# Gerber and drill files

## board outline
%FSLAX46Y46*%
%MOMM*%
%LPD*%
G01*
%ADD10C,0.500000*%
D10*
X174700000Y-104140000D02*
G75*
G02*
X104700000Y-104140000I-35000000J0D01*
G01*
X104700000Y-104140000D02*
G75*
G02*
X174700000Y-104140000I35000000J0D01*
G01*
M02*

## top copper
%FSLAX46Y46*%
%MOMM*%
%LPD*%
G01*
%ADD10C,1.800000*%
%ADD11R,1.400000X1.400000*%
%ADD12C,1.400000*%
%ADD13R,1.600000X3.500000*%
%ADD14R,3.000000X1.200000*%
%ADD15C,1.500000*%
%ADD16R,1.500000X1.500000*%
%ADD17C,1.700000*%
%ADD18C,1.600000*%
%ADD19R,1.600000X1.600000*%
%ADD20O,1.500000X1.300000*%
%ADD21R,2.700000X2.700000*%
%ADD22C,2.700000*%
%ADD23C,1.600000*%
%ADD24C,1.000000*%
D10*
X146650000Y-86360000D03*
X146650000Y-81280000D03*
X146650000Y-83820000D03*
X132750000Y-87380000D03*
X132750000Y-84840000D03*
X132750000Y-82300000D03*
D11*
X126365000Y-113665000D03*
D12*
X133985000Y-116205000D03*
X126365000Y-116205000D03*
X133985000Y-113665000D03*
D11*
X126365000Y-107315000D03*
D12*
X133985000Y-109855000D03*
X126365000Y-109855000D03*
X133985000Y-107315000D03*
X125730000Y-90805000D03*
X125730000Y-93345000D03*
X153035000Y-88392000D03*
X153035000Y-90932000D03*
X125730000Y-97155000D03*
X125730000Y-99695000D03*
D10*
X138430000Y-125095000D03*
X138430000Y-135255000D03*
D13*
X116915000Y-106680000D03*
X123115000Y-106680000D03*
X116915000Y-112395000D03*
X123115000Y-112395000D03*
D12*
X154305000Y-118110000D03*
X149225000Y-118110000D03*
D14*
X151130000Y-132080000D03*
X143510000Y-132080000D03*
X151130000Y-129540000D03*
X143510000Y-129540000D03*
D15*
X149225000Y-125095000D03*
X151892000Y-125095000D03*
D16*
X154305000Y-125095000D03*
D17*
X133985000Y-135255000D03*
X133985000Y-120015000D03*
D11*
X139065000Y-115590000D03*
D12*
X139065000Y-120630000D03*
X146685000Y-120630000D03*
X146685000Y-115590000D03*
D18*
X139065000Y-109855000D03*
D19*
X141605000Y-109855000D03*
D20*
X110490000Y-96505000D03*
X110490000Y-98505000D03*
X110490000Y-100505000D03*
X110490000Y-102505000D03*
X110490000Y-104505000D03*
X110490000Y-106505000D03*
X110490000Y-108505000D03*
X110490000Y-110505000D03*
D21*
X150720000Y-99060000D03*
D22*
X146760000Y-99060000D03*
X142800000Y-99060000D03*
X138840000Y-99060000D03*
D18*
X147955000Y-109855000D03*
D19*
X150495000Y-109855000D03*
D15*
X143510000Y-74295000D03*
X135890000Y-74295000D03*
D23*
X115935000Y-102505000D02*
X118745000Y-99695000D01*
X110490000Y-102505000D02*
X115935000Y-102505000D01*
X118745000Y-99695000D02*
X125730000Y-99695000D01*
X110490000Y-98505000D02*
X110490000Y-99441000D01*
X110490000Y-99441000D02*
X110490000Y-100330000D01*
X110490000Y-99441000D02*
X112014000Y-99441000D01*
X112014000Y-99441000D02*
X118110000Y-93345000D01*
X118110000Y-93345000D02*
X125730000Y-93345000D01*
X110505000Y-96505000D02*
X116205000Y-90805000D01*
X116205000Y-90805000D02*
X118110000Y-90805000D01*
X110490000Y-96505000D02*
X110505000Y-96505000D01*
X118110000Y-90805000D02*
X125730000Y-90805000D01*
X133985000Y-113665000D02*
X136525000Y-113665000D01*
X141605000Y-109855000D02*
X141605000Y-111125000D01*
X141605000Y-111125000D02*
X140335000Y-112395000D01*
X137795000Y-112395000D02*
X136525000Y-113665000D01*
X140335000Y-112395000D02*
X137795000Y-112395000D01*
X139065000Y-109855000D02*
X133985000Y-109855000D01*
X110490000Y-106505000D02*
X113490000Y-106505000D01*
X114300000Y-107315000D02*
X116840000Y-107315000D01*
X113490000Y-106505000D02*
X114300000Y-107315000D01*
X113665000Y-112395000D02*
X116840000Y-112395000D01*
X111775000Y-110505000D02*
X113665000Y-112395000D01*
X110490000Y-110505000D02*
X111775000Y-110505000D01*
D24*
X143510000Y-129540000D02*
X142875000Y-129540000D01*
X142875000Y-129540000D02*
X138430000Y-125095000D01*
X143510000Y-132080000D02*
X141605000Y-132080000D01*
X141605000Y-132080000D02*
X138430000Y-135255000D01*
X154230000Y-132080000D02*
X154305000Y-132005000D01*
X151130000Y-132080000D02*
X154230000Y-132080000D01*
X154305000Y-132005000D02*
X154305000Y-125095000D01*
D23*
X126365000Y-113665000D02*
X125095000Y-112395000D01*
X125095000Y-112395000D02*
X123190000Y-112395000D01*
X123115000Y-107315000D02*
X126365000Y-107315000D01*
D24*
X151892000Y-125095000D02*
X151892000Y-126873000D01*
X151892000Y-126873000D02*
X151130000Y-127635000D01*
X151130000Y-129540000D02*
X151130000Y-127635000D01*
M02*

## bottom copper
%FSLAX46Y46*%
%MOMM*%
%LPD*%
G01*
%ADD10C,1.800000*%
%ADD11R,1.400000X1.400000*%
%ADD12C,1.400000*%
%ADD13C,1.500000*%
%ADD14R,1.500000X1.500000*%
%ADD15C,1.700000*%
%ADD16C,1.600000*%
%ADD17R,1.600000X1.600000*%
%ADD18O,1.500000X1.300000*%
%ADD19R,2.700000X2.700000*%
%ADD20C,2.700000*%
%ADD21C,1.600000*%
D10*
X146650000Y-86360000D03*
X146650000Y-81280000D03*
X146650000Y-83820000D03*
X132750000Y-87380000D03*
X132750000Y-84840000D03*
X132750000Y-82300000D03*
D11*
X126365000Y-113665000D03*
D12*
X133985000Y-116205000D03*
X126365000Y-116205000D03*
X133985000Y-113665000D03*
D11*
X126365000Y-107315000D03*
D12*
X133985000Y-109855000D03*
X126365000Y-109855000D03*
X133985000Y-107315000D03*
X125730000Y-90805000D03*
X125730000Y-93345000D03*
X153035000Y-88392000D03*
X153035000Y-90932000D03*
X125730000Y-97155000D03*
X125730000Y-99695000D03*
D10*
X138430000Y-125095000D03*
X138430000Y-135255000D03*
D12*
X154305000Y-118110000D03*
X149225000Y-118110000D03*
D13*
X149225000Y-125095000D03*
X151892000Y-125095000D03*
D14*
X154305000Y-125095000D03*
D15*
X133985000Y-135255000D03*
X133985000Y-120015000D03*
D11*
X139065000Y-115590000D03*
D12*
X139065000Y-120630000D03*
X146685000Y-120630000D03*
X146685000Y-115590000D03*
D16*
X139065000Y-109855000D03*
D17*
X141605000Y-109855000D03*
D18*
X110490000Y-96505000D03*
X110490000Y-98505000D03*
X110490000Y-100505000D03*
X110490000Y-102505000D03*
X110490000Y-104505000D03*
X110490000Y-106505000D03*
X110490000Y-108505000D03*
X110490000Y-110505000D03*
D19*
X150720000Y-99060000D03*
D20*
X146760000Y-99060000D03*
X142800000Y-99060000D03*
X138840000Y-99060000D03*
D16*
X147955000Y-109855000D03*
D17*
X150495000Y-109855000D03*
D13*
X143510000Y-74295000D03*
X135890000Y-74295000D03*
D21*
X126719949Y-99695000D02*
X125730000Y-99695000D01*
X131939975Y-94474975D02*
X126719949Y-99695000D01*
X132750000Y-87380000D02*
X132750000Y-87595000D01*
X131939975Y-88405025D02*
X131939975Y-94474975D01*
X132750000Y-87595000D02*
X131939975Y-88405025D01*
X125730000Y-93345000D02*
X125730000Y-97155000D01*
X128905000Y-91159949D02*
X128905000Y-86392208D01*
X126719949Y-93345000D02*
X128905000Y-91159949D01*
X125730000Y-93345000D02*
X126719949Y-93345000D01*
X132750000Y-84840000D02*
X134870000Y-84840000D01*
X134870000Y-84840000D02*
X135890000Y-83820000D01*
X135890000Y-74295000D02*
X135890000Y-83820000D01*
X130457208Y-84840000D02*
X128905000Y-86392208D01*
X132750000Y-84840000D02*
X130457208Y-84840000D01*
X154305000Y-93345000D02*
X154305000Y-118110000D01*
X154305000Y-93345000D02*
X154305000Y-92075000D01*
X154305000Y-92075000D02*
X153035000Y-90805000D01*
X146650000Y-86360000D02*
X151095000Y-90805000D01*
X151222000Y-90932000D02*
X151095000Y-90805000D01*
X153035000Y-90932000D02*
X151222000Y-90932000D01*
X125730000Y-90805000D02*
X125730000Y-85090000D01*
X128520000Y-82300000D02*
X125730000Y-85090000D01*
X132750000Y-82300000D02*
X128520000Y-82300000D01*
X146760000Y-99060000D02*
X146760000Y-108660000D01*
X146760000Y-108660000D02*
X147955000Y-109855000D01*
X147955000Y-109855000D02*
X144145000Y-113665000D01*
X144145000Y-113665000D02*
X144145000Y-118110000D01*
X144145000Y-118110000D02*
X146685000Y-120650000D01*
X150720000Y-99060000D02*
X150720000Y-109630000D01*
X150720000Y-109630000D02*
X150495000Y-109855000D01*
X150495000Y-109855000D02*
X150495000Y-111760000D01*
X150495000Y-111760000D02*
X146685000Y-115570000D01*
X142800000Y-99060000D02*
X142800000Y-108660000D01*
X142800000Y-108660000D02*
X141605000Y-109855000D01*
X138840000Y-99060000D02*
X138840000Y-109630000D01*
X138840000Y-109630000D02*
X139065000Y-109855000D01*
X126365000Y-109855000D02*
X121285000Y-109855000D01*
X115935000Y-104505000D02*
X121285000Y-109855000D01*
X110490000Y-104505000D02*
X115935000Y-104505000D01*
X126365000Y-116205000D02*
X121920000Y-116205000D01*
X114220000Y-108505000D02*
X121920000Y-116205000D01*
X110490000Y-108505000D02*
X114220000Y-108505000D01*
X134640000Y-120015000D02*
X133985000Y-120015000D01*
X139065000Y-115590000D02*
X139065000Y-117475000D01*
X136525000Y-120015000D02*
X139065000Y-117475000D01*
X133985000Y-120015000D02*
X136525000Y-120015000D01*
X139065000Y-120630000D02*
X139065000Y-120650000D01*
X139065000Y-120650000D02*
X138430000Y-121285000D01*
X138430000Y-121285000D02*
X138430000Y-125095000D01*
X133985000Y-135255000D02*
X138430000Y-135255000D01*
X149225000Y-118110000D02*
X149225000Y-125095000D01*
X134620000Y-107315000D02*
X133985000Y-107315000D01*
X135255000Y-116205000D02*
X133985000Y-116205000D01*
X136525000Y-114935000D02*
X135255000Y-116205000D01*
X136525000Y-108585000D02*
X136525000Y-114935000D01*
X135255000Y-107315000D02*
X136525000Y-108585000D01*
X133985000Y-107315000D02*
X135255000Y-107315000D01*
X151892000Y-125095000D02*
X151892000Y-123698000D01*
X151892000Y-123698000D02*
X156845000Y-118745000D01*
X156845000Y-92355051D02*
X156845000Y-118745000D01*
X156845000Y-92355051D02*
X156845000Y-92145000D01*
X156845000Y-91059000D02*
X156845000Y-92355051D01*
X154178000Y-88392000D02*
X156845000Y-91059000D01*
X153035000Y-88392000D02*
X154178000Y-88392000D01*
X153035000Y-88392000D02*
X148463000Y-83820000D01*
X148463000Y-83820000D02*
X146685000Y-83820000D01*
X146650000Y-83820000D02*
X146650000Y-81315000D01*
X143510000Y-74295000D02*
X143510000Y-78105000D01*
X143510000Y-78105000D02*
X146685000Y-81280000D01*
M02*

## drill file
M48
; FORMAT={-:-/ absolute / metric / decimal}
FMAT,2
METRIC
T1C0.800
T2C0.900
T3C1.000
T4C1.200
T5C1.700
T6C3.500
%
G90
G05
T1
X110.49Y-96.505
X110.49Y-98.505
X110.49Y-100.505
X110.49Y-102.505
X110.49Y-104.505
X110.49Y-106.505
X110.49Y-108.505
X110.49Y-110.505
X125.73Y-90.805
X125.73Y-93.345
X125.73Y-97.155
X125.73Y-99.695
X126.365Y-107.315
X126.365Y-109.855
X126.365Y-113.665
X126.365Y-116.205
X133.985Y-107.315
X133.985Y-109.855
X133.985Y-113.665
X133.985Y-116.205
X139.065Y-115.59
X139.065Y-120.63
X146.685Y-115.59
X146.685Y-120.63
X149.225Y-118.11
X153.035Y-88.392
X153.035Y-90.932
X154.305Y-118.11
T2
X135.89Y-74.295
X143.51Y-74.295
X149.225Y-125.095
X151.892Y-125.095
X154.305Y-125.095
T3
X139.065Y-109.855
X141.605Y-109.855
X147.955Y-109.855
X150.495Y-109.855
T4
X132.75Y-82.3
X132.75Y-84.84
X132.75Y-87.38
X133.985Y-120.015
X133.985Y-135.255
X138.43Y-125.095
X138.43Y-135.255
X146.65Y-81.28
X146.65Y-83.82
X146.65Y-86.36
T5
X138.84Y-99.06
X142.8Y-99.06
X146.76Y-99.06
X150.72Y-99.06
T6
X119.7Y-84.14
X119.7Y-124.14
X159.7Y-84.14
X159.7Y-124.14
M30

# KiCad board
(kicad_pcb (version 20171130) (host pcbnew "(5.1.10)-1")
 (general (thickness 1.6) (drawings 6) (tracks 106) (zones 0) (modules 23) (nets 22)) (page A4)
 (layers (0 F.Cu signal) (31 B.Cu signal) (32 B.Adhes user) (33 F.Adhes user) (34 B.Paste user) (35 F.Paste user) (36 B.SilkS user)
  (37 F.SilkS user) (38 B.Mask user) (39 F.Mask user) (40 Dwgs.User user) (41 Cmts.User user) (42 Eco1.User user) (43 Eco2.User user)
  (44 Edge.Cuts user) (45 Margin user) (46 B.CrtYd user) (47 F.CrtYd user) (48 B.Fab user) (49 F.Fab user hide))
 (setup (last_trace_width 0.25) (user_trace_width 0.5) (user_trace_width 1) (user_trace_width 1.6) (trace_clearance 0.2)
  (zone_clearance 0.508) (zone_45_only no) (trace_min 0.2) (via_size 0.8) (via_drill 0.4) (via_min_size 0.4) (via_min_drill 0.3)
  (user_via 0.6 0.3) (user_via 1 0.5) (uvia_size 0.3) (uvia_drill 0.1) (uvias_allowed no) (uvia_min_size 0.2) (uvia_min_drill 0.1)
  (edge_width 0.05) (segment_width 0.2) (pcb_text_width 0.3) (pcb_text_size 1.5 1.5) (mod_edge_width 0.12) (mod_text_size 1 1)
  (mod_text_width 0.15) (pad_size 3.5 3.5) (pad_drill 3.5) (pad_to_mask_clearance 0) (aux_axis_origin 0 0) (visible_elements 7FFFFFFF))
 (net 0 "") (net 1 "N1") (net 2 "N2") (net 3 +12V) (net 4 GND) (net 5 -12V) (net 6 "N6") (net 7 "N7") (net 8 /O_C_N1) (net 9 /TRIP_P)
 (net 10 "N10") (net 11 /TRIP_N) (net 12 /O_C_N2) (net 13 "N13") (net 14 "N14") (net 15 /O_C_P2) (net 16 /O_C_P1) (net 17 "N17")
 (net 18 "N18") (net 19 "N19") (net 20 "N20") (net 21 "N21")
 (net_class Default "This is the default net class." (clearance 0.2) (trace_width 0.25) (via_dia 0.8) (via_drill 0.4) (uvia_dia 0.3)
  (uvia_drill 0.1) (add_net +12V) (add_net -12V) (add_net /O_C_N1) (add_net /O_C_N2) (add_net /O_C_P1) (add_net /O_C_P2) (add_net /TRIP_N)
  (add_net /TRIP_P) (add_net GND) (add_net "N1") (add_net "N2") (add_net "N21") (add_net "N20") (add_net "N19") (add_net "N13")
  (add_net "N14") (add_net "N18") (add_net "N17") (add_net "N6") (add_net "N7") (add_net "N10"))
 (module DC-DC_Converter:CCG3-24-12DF (layer F.Cu) (at 139.7 83.82)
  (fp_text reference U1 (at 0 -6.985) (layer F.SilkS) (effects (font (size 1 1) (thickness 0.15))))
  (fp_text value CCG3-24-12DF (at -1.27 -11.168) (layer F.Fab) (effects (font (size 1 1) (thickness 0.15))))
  (pad 3 thru_hole circle (at 6.95 2.54) (size 1.8 1.8) (drill 1.2) (layers *.Cu *.Mask) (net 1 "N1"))
  (pad 1 thru_hole circle (at 6.95 -2.54) (size 1.8 1.8) (drill 1.2) (layers *.Cu *.Mask) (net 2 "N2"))
  (pad 2 thru_hole circle (at 6.95 0) (size 1.8 1.8) (drill 1.2) (layers *.Cu *.Mask) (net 2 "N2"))
  (pad 6 thru_hole circle (at -6.95 3.56) (size 1.8 1.8) (drill 1.2) (layers *.Cu *.Mask) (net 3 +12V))
  (pad 5 thru_hole circle (at -6.95 1.02) (size 1.8 1.8) (drill 1.2) (layers *.Cu *.Mask) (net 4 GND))
  (pad 4 thru_hole circle (at -6.95 -1.52) (size 1.8 1.8) (drill 1.2) (layers *.Cu *.Mask) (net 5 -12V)))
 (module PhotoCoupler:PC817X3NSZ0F (layer F.Cu) (at 126.365 113.665)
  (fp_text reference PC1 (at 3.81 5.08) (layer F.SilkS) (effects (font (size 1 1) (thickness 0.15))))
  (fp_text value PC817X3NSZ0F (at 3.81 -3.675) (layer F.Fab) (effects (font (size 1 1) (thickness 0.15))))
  (pad 1 thru_hole rect (at 0 0) (size 1.4 1.4) (drill 0.8) (layers *.Cu *.Mask) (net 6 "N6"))
  (pad 3 thru_hole circle (at 7.62 2.54) (size 1.4 1.4) (drill 0.8) (layers *.Cu *.Mask) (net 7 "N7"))
  (pad 2 thru_hole circle (at 0 2.54) (size 1.4 1.4) (drill 0.8) (layers *.Cu *.Mask) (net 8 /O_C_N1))
  (pad 4 thru_hole circle (at 7.62 0) (size 1.4 1.4) (drill 0.8) (layers *.Cu *.Mask) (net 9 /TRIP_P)))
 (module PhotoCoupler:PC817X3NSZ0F (layer F.Cu) (at 126.365 107.315)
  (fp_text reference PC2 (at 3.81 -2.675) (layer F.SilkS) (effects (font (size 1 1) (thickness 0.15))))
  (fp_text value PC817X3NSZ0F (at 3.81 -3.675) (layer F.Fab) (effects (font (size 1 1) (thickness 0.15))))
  (pad 1 thru_hole rect (at 0 0) (size 1.4 1.4) (drill 0.8) (layers *.Cu *.Mask) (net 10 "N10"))
  (pad 3 thru_hole circle (at 7.62 2.54) (size 1.4 1.4) (drill 0.8) (layers *.Cu *.Mask) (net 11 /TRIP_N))
  (pad 2 thru_hole circle (at 0 2.54) (size 1.4 1.4) (drill 0.8) (layers *.Cu *.Mask) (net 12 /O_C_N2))
  (pad 4 thru_hole circle (at 7.62 0) (size 1.4 1.4) (drill 0.8) (layers *.Cu *.Mask) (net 7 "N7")))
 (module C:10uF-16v (layer F.Cu) (at 125.73 92.075 90)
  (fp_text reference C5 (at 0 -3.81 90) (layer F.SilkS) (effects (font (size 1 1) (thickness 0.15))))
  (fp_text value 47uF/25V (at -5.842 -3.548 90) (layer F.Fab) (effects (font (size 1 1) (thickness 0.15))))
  (pad 2 thru_hole circle (at 1.27 0 90) (size 1.4 1.4) (drill 0.8) (layers *.Cu *.Mask) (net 5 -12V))
  (pad 1 thru_hole circle (at -1.27 0 90) (size 1.4 1.4) (drill 0.8) (layers *.Cu *.Mask) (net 4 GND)))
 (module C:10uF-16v (layer F.Cu) (at 153.035 89.662 90)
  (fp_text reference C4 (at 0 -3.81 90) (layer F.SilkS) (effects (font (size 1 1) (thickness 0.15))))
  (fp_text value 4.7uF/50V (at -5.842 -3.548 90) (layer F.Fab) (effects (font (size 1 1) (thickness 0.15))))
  (pad 2 thru_hole circle (at 1.27 0 90) (size 1.4 1.4) (drill 0.8) (layers *.Cu *.Mask) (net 2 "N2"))
  (pad 1 thru_hole circle (at -1.27 0 90) (size 1.4 1.4) (drill 0.8) (layers *.Cu *.Mask) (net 1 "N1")))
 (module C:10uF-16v (layer F.Cu) (at 125.73 98.425 90)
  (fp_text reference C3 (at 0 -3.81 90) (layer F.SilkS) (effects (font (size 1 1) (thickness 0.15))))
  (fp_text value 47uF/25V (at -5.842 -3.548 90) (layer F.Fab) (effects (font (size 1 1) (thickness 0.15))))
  (pad 2 thru_hole circle (at 1.27 0 90) (size 1.4 1.4) (drill 0.8) (layers *.Cu *.Mask) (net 4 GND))
  (pad 1 thru_hole circle (at -1.27 0 90) (size 1.4 1.4) (drill 0.8) (layers *.Cu *.Mask) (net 3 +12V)))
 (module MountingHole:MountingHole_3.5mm (layer F.Cu) (at 119.7 84.14)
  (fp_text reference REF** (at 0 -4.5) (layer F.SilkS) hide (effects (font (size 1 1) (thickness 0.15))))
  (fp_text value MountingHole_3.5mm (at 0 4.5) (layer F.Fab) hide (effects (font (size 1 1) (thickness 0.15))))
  (pad 1 np_thru_hole circle (at 0 0) (size 3.5 3.5) (drill 3.5) (layers *.Cu *.Mask)))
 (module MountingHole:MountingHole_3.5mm (layer F.Cu) (at 119.7 124.14)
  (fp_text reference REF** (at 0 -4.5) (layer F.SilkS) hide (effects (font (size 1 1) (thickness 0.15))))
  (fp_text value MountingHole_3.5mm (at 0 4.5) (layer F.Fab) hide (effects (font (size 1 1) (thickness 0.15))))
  (pad 1 np_thru_hole circle (at 0 0) (size 3.5 3.5) (drill 3.5) (layers *.Cu *.Mask)))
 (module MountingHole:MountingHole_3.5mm (layer F.Cu) (at 159.7 124.14)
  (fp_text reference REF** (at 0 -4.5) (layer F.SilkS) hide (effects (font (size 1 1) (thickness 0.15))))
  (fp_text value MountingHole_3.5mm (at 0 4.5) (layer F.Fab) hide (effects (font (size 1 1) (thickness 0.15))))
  (pad 1 np_thru_hole circle (at 0 0) (size 3.5 3.5) (drill 3.5) (layers *.Cu *.Mask)))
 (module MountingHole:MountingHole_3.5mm (layer F.Cu) (at 159.7 84.14)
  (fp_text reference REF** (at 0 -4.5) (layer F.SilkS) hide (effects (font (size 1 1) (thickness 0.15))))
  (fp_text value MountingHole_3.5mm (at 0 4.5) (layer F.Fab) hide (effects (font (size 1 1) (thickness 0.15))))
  (pad 1 np_thru_hole circle (at 0 0) (size 3.5 3.5) (drill 3.5) (layers *.Cu *.Mask)))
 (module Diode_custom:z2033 (layer F.Cu) (at 138.43 130.175 90)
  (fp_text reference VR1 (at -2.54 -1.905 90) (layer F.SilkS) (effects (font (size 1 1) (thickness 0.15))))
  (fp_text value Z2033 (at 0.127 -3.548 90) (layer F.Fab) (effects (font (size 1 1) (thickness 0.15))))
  (pad 2 thru_hole circle (at 5.08 0 90) (size 1.8 1.8) (drill 1.2) (layers *.Cu *.Mask) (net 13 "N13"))
  (pad 1 thru_hole circle (at -5.08 0 90) (size 1.8 1.8) (drill 1.2) (layers *.Cu *.Mask) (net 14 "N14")))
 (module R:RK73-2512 (layer F.Cu) (at 120.015 106.68)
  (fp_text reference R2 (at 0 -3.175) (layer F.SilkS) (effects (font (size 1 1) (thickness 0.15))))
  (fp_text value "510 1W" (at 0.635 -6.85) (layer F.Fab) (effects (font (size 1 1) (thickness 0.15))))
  (pad 1 smd rect (at -3.1 0) (size 1.6 3.5) (layers F.Cu F.Paste F.Mask) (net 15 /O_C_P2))
  (pad 2 smd rect (at 3.1 0) (size 1.6 3.5) (layers F.Cu F.Paste F.Mask) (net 10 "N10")))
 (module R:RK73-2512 (layer F.Cu) (at 120.015 112.395)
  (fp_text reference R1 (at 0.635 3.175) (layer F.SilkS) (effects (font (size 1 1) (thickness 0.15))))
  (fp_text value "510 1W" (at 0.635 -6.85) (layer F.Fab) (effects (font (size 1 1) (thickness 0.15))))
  (pad 1 smd rect (at -3.1 0) (size 1.6 3.5) (layers F.Cu F.Paste F.Mask) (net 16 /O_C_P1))
  (pad 2 smd rect (at 3.1 0) (size 1.6 3.5) (layers F.Cu F.Paste F.Mask) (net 6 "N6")))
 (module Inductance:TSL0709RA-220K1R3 (layer F.Cu) (at 151.765 118.11)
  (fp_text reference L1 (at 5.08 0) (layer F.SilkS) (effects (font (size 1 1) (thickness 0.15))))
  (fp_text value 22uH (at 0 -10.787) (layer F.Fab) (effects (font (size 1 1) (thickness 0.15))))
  (pad 2 thru_hole circle (at 2.54 0) (size 1.4 1.4) (drill 0.8) (layers *.Cu *.Mask) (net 1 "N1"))
  (pad 1 thru_hole circle (at -2.54 0) (size 1.4 1.4) (drill 0.8) (layers *.Cu *.Mask) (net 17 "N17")))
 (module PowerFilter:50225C (layer F.Cu) (at 147.32 130.81)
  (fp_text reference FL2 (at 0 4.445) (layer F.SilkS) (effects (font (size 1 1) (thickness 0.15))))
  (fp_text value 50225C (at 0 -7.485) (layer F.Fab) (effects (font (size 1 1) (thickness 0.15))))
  (pad 3 smd rect (at 3.81 1.27) (size 3 1.2) (layers F.Cu F.Paste F.Mask) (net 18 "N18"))
  (pad 2 smd rect (at -3.81 1.27) (size 3 1.2) (layers F.Cu F.Paste F.Mask) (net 14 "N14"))
  (pad 4 smd rect (at 3.81 -1.27) (size 3 1.2) (layers F.Cu F.Paste F.Mask) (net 2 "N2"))
  (pad 1 smd rect (at -3.81 -1.27) (size 3 1.2) (layers F.Cu F.Paste F.Mask) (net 13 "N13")))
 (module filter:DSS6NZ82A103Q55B (layer F.Cu) (at 151.765 125.095 180)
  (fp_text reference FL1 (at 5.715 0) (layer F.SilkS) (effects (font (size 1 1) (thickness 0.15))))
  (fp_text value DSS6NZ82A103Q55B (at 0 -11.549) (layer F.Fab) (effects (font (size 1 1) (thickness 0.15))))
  (pad 3 thru_hole circle (at 2.54 0 180) (size 1.5 1.5) (drill 0.9) (layers *.Cu *.Mask) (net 17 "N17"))
  (pad 2 thru_hole circle (at -0.127 0 180) (size 1.5 1.5) (drill 0.9) (layers *.Cu *.Mask) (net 2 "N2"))
  (pad 1 thru_hole rect (at -2.54 0 180) (size 1.5 1.5) (drill 0.9) (layers *.Cu *.Mask) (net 18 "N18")))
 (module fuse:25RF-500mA (layer F.Cu) (at 133.985 127.635 270)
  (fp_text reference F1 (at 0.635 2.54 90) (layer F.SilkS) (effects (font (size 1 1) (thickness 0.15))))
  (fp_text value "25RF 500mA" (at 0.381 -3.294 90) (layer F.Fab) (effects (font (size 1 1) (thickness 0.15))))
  (pad 2 thru_hole circle (at 7.62 0 270) (size 1.7 1.7) (drill 1.2) (layers *.Cu *.Mask) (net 14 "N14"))
  (pad 1 thru_hole circle (at -7.62 0 270) (size 1.7 1.7) (drill 1.2) (layers *.Cu *.Mask) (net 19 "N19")))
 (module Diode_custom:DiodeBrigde (layer F.Cu) (at 142.875 118.11)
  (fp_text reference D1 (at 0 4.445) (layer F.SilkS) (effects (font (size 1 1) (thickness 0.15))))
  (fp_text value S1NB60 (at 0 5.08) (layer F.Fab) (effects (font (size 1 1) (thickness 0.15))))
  (pad 1 thru_hole rect (at -3.81 -2.52) (size 1.4 1.4) (drill 0.8) (layers *.Cu *.Mask) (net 19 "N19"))
  (pad 4 thru_hole circle (at -3.81 2.52) (size 1.4 1.4) (drill 0.8) (layers *.Cu *.Mask) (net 13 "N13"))
  (pad 3 thru_hole circle (at 3.81 2.52) (size 1.4 1.4) (drill 0.8) (layers *.Cu *.Mask) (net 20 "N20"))
  (pad 2 thru_hole circle (at 3.81 -2.52) (size 1.4 1.4) (drill 0.8) (layers *.Cu *.Mask) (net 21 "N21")))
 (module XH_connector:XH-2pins (layer F.Cu) (at 140.208 109.855 270)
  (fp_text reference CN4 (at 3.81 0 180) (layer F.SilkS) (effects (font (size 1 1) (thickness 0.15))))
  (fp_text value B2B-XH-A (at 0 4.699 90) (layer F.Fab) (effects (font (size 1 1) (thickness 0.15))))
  (pad 2 thru_hole circle (at 0 1.143 270) (size 1.6 1.6) (drill 1) (layers *.Cu *.Mask) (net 11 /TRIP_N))
  (pad 1 thru_hole rect (at 0 -1.397 270) (size 1.6 1.6) (drill 1) (layers *.Cu *.Mask) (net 9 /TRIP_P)))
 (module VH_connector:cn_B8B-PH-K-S (layer F.Cu) (at 110.49 103.505 90)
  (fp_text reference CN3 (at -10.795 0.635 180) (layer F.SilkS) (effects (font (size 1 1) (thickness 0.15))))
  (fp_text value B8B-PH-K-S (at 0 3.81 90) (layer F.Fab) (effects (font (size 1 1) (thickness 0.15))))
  (pad 8 thru_hole oval (at 7 0 90) (size 1.3 1.5) (drill 0.8) (layers *.Cu *.Mask) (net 5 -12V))
  (pad 7 thru_hole oval (at 5 0 90) (size 1.3 1.5) (drill 0.8) (layers *.Cu *.Mask) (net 4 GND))
  (pad 6 thru_hole oval (at 3 0 90) (size 1.3 1.5) (drill 0.8) (layers *.Cu *.Mask) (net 4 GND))
  (pad 5 thru_hole oval (at 1 0 90) (size 1.3 1.5) (drill 0.8) (layers *.Cu *.Mask) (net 3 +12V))
  (pad 4 thru_hole oval (at -1 0 90) (size 1.3 1.5) (drill 0.8) (layers *.Cu *.Mask) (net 12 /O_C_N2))
  (pad 3 thru_hole oval (at -3 0 90) (size 1.3 1.5) (drill 0.8) (layers *.Cu *.Mask) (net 15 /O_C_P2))
  (pad 2 thru_hole oval (at -5 0 90) (size 1.3 1.5) (drill 0.8) (layers *.Cu *.Mask) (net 8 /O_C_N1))
  (pad 1 thru_hole oval (at -7 0 90) (size 1.3 1.5) (drill 0.8) (layers *.Cu *.Mask) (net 16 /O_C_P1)))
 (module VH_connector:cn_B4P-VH (layer F.Cu) (at 144.78 99.06 180)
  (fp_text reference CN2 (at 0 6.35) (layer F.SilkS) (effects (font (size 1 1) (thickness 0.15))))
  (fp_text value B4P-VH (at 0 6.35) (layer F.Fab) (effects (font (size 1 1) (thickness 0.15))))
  (pad 1 thru_hole rect (at -5.94 0 180) (size 2.7 2.7) (drill 1.7) (layers *.Cu *.Mask) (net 21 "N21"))
  (pad 2 thru_hole circle (at -1.98 0 180) (size 2.7 2.7) (drill 1.7) (layers *.Cu *.Mask) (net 20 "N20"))
  (pad 3 thru_hole circle (at 1.98 0 180) (size 2.7 2.7) (drill 1.7) (layers *.Cu *.Mask) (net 9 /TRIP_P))
  (pad 4 thru_hole circle (at 5.94 0 180) (size 2.7 2.7) (drill 1.7) (layers *.Cu *.Mask) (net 11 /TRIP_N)))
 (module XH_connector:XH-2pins (layer F.Cu) (at 149.098 109.855 270)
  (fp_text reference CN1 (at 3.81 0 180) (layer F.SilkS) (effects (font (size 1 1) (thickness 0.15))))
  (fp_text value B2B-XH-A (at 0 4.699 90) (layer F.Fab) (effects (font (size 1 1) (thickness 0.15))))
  (pad 2 thru_hole circle (at 0 1.143 270) (size 1.6 1.6) (drill 1) (layers *.Cu *.Mask) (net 20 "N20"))
  (pad 1 thru_hole rect (at 0 -1.397 270) (size 1.6 1.6) (drill 1) (layers *.Cu *.Mask) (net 21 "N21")))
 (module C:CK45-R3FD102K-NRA (layer F.Cu) (at 139.7 74.295)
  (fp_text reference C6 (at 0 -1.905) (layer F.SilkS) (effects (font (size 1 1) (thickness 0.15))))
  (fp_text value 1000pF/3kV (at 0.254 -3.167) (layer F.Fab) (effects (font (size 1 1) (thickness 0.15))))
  (pad 2 thru_hole circle (at 3.81 0) (size 1.5 1.5) (drill 0.9) (layers *.Cu *.Mask) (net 2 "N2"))
  (pad 1 thru_hole circle (at -3.81 0) (size 1.5 1.5) (drill 0.9) (layers *.Cu *.Mask) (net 4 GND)))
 (gr_circle (center 139.7 104.14) (end 174.7 104.14) (layer Edge.Cuts) (width 0.5))
 (segment (start 115.935 102.505) (end 118.745 99.695) (width 1.6) (layer F.Cu) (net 3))
 (segment (start 110.49 102.505) (end 115.935 102.505) (width 1.6) (layer F.Cu) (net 3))
 (segment (start 126.719949 99.695) (end 125.73 99.695) (width 1.6) (layer B.Cu) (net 3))
 (segment (start 118.745 99.695) (end 125.73 99.695) (width 1.6) (layer F.Cu) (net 3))
 (segment (start 131.939975 94.474975) (end 126.719949 99.695) (width 1.6) (layer B.Cu) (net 3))
 (segment (start 132.75 87.38) (end 132.75 87.595) (width 1.6) (layer B.Cu) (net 3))
 (segment (start 131.939975 88.405025) (end 131.939975 94.474975) (width 1.6) (layer B.Cu) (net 3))
 (segment (start 132.75 87.595) (end 131.939975 88.405025) (width 1.6) (layer B.Cu) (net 3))
 (segment (start 110.49 98.505) (end 110.49 99.441) (width 1.6) (layer F.Cu) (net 4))
 (segment (start 110.49 99.441) (end 110.49 100.33) (width 1.6) (layer F.Cu) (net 4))
 (segment (start 125.73 93.345) (end 125.73 97.155) (width 1.6) (layer B.Cu) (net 4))
 (segment (start 110.49 99.441) (end 112.014 99.441) (width 1.6) (layer F.Cu) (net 4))
 (segment (start 112.014 99.441) (end 118.11 93.345) (width 1.6) (layer F.Cu) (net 4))
 (segment (start 118.11 93.345) (end 125.73 93.345) (width 1.6) (layer F.Cu) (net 4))
 (segment (start 128.905 91.159949) (end 128.905 86.392208) (width 1.6) (layer B.Cu) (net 4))
 (segment (start 126.719949 93.345) (end 128.905 91.159949) (width 1.6) (layer B.Cu) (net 4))
 (segment (start 125.73 93.345) (end 126.719949 93.345) (width 1.6) (layer B.Cu) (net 4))
 (segment (start 132.75 84.84) (end 134.87 84.84) (width 1.6) (layer B.Cu) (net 4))
 (segment (start 134.87 84.84) (end 135.89 83.82) (width 1.6) (layer B.Cu) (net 4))
 (segment (start 135.89 74.295) (end 135.89 83.82) (width 1.6) (layer B.Cu) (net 4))
 (segment (start 130.457208 84.84) (end 128.905 86.392208) (width 1.6) (layer B.Cu) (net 4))
 (segment (start 132.75 84.84) (end 130.457208 84.84) (width 1.6) (layer B.Cu) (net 4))
 (segment (start 154.305 93.345) (end 154.305 118.11) (width 1.6) (layer B.Cu) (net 1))
 (segment (start 154.305 93.345) (end 154.305 92.075) (width 1.6) (layer B.Cu) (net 1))
 (segment (start 154.305 92.075) (end 153.035 90.805) (width 1.6) (layer B.Cu) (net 1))
 (segment (start 146.65 86.36) (end 151.095 90.805) (width 1.6) (layer B.Cu) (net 1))
 (segment (start 151.222 90.932) (end 151.095 90.805) (width 1.6) (layer B.Cu) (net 1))
 (segment (start 153.035 90.932) (end 151.222 90.932) (width 1.6) (layer B.Cu) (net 1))
 (segment (start 110.505 96.505) (end 116.205 90.805) (width 1.6) (layer F.Cu) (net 5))
 (segment (start 116.205 90.805) (end 118.11 90.805) (width 1.6) (layer F.Cu) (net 5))
 (segment (start 110.49 96.505) (end 110.505 96.505) (width 1.6) (layer F.Cu) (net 5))
 (segment (start 118.11 90.805) (end 125.73 90.805) (width 1.6) (layer F.Cu) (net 5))
 (segment (start 125.73 90.805) (end 125.73 85.09) (width 1.6) (layer B.Cu) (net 5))
 (segment (start 128.52 82.3) (end 125.73 85.09) (width 1.6) (layer B.Cu) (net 5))
 (segment (start 132.75 82.3) (end 128.52 82.3) (width 1.6) (layer B.Cu) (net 5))
 (segment (start 146.76 99.06) (end 146.76 108.66) (width 1.6) (layer B.Cu) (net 20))
 (segment (start 146.76 108.66) (end 147.955 109.855) (width 1.6) (layer B.Cu) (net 20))
 (segment (start 147.955 109.855) (end 144.145 113.665) (width 1.6) (layer B.Cu) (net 20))
 (segment (start 144.145 113.665) (end 144.145 118.11) (width 1.6) (layer B.Cu) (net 20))
 (segment (start 144.145 118.11) (end 146.685 120.65) (width 1.6) (layer B.Cu) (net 20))
 (segment (start 150.72 99.06) (end 150.72 109.63) (width 1.6) (layer B.Cu) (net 21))
 (segment (start 150.72 109.63) (end 150.495 109.855) (width 1.6) (layer B.Cu) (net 21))
 (segment (start 150.495 109.855) (end 150.495 111.76) (width 1.6) (layer B.Cu) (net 21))
 (segment (start 150.495 111.76) (end 146.685 115.57) (width 1.6) (layer B.Cu) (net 21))
 (segment (start 142.8 99.06) (end 142.8 108.66) (width 1.6) (layer B.Cu) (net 9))
 (segment (start 142.8 108.66) (end 141.605 109.855) (width 1.6) (layer B.Cu) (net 9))
 (segment (start 133.985 113.665) (end 136.525 113.665) (width 1.6) (layer F.Cu) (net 9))
 (segment (start 141.605 109.855) (end 141.605 111.125) (width 1.6) (layer F.Cu) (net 9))
 (segment (start 141.605 111.125) (end 140.335 112.395) (width 1.6) (layer F.Cu) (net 9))
 (segment (start 137.795 112.395) (end 136.525 113.665) (width 1.6) (layer F.Cu) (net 9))
 (segment (start 140.335 112.395) (end 137.795 112.395) (width 1.6) (layer F.Cu) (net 9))
 (segment (start 138.84 99.06) (end 138.84 109.63) (width 1.6) (layer B.Cu) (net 11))
 (segment (start 138.84 109.63) (end 139.065 109.855) (width 1.6) (layer B.Cu) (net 11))
 (segment (start 139.065 109.855) (end 133.985 109.855) (width 1.6) (layer F.Cu) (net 11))
 (segment (start 126.365 109.855) (end 121.285 109.855) (width 1.6) (layer B.Cu) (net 12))
 (segment (start 115.935 104.505) (end 121.285 109.855) (width 1.6) (layer B.Cu) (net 12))
 (segment (start 110.49 104.505) (end 115.935 104.505) (width 1.6) (layer B.Cu) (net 12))
 (segment (start 110.49 106.505) (end 113.49 106.505) (width 1.6) (layer F.Cu) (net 15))
 (segment (start 114.3 107.315) (end 116.84 107.315) (width 1.6) (layer F.Cu) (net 15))
 (segment (start 113.49 106.505) (end 114.3 107.315) (width 1.6) (layer F.Cu) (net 15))
 (segment (start 126.365 116.205) (end 121.92 116.205) (width 1.6) (layer B.Cu) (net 8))
 (segment (start 114.22 108.505) (end 121.92 116.205) (width 1.6) (layer B.Cu) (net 8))
 (segment (start 110.49 108.505) (end 114.22 108.505) (width 1.6) (layer B.Cu) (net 8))
 (segment (start 113.665 112.395) (end 116.84 112.395) (width 1.6) (layer F.Cu) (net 16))
 (segment (start 111.775 110.505) (end 113.665 112.395) (width 1.6) (layer F.Cu) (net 16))
 (segment (start 110.49 110.505) (end 111.775 110.505) (width 1.6) (layer F.Cu) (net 16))
 (segment (start 134.64 120.015) (end 133.985 120.015) (width 1.6) (layer B.Cu) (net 19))
 (segment (start 139.065 115.59) (end 139.065 117.475) (width 1.6) (layer B.Cu) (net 19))
 (segment (start 136.525 120.015) (end 139.065 117.475) (width 1.6) (layer B.Cu) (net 19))
 (segment (start 133.985 120.015) (end 136.525 120.015) (width 1.6) (layer B.Cu) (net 19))
 (segment (start 143.51 129.54) (end 142.875 129.54) (width 1) (layer F.Cu) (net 13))
 (segment (start 142.875 129.54) (end 138.43 125.095) (width 1) (layer F.Cu) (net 13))
 (segment (start 139.065 120.63) (end 139.065 120.65) (width 1.6) (layer B.Cu) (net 13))
 (segment (start 139.065 120.65) (end 138.43 121.285) (width 1.6) (layer B.Cu) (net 13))
 (segment (start 138.43 121.285) (end 138.43 125.095) (width 1.6) (layer B.Cu) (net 13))
 (segment (start 143.51 132.08) (end 141.605 132.08) (width 1) (layer F.Cu) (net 14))
 (segment (start 141.605 132.08) (end 138.43 135.255) (width 1) (layer F.Cu) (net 14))
 (segment (start 133.985 135.255) (end 138.43 135.255) (width 1.6) (layer B.Cu) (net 14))
 (segment (start 149.225 118.11) (end 149.225 125.095) (width 1.6) (layer B.Cu) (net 17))
 (segment (start 154.23 132.08) (end 154.305 132.005) (width 1) (layer F.Cu) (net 18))
 (segment (start 151.13 132.08) (end 154.23 132.08) (width 1) (layer F.Cu) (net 18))
 (segment (start 154.305 132.005) (end 154.305 125.095) (width 1) (layer F.Cu) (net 18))
 (segment (start 126.365 113.665) (end 125.095 112.395) (width 1.6) (layer F.Cu) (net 6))
 (segment (start 125.095 112.395) (end 123.19 112.395) (width 1.6) (layer F.Cu) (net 6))
 (segment (start 134.62 107.315) (end 133.985 107.315) (width 1.6) (layer B.Cu) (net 7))
 (segment (start 135.255 116.205) (end 133.985 116.205) (width 1.6) (layer B.Cu) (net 7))
 (segment (start 136.525 114.935) (end 135.255 116.205) (width 1.6) (layer B.Cu) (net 7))
 (segment (start 136.525 108.585) (end 136.525 114.935) (width 1.6) (layer B.Cu) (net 7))
 (segment (start 135.255 107.315) (end 136.525 108.585) (width 1.6) (layer B.Cu) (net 7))
 (segment (start 133.985 107.315) (end 135.255 107.315) (width 1.6) (layer B.Cu) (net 7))
 (segment (start 123.115 107.315) (end 126.365 107.315) (width 1.6) (layer F.Cu) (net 10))
 (segment (start 151.892 125.095) (end 151.892 123.698) (width 1.6) (layer B.Cu) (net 2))
 (segment (start 151.892 123.698) (end 156.845 118.745) (width 1.6) (layer B.Cu) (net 2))
 (segment (start 156.845 92.355051) (end 156.845 118.745) (width 1.6) (layer B.Cu) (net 2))
 (segment (start 151.892 125.095) (end 151.892 126.873) (width 1) (layer F.Cu) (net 2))
 (segment (start 151.892 126.873) (end 151.13 127.635) (width 1) (layer F.Cu) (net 2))
 (segment (start 151.13 129.54) (end 151.13 127.635) (width 1) (layer F.Cu) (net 2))
 (segment (start 156.845 92.355051) (end 156.845 92.145) (width 1.6) (layer B.Cu) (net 2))
 (segment (start 156.845 91.059) (end 156.845 92.355051) (width 1.6) (layer B.Cu) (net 2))
 (segment (start 154.178 88.392) (end 156.845 91.059) (width 1.6) (layer B.Cu) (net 2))
 (segment (start 153.035 88.392) (end 154.178 88.392) (width 1.6) (layer B.Cu) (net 2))
 (segment (start 153.035 88.392) (end 148.463 83.82) (width 1.6) (layer B.Cu) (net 2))
 (segment (start 148.463 83.82) (end 146.685 83.82) (width 1.6) (layer B.Cu) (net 2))
 (segment (start 146.65 83.82) (end 146.65 81.315) (width 1.6) (layer B.Cu) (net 2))
 (segment (start 143.51 74.295) (end 143.51 78.105) (width 1.6) (layer B.Cu) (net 2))
 (segment (start 143.51 78.105) (end 146.685 81.28) (width 1.6) (layer B.Cu) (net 2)))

